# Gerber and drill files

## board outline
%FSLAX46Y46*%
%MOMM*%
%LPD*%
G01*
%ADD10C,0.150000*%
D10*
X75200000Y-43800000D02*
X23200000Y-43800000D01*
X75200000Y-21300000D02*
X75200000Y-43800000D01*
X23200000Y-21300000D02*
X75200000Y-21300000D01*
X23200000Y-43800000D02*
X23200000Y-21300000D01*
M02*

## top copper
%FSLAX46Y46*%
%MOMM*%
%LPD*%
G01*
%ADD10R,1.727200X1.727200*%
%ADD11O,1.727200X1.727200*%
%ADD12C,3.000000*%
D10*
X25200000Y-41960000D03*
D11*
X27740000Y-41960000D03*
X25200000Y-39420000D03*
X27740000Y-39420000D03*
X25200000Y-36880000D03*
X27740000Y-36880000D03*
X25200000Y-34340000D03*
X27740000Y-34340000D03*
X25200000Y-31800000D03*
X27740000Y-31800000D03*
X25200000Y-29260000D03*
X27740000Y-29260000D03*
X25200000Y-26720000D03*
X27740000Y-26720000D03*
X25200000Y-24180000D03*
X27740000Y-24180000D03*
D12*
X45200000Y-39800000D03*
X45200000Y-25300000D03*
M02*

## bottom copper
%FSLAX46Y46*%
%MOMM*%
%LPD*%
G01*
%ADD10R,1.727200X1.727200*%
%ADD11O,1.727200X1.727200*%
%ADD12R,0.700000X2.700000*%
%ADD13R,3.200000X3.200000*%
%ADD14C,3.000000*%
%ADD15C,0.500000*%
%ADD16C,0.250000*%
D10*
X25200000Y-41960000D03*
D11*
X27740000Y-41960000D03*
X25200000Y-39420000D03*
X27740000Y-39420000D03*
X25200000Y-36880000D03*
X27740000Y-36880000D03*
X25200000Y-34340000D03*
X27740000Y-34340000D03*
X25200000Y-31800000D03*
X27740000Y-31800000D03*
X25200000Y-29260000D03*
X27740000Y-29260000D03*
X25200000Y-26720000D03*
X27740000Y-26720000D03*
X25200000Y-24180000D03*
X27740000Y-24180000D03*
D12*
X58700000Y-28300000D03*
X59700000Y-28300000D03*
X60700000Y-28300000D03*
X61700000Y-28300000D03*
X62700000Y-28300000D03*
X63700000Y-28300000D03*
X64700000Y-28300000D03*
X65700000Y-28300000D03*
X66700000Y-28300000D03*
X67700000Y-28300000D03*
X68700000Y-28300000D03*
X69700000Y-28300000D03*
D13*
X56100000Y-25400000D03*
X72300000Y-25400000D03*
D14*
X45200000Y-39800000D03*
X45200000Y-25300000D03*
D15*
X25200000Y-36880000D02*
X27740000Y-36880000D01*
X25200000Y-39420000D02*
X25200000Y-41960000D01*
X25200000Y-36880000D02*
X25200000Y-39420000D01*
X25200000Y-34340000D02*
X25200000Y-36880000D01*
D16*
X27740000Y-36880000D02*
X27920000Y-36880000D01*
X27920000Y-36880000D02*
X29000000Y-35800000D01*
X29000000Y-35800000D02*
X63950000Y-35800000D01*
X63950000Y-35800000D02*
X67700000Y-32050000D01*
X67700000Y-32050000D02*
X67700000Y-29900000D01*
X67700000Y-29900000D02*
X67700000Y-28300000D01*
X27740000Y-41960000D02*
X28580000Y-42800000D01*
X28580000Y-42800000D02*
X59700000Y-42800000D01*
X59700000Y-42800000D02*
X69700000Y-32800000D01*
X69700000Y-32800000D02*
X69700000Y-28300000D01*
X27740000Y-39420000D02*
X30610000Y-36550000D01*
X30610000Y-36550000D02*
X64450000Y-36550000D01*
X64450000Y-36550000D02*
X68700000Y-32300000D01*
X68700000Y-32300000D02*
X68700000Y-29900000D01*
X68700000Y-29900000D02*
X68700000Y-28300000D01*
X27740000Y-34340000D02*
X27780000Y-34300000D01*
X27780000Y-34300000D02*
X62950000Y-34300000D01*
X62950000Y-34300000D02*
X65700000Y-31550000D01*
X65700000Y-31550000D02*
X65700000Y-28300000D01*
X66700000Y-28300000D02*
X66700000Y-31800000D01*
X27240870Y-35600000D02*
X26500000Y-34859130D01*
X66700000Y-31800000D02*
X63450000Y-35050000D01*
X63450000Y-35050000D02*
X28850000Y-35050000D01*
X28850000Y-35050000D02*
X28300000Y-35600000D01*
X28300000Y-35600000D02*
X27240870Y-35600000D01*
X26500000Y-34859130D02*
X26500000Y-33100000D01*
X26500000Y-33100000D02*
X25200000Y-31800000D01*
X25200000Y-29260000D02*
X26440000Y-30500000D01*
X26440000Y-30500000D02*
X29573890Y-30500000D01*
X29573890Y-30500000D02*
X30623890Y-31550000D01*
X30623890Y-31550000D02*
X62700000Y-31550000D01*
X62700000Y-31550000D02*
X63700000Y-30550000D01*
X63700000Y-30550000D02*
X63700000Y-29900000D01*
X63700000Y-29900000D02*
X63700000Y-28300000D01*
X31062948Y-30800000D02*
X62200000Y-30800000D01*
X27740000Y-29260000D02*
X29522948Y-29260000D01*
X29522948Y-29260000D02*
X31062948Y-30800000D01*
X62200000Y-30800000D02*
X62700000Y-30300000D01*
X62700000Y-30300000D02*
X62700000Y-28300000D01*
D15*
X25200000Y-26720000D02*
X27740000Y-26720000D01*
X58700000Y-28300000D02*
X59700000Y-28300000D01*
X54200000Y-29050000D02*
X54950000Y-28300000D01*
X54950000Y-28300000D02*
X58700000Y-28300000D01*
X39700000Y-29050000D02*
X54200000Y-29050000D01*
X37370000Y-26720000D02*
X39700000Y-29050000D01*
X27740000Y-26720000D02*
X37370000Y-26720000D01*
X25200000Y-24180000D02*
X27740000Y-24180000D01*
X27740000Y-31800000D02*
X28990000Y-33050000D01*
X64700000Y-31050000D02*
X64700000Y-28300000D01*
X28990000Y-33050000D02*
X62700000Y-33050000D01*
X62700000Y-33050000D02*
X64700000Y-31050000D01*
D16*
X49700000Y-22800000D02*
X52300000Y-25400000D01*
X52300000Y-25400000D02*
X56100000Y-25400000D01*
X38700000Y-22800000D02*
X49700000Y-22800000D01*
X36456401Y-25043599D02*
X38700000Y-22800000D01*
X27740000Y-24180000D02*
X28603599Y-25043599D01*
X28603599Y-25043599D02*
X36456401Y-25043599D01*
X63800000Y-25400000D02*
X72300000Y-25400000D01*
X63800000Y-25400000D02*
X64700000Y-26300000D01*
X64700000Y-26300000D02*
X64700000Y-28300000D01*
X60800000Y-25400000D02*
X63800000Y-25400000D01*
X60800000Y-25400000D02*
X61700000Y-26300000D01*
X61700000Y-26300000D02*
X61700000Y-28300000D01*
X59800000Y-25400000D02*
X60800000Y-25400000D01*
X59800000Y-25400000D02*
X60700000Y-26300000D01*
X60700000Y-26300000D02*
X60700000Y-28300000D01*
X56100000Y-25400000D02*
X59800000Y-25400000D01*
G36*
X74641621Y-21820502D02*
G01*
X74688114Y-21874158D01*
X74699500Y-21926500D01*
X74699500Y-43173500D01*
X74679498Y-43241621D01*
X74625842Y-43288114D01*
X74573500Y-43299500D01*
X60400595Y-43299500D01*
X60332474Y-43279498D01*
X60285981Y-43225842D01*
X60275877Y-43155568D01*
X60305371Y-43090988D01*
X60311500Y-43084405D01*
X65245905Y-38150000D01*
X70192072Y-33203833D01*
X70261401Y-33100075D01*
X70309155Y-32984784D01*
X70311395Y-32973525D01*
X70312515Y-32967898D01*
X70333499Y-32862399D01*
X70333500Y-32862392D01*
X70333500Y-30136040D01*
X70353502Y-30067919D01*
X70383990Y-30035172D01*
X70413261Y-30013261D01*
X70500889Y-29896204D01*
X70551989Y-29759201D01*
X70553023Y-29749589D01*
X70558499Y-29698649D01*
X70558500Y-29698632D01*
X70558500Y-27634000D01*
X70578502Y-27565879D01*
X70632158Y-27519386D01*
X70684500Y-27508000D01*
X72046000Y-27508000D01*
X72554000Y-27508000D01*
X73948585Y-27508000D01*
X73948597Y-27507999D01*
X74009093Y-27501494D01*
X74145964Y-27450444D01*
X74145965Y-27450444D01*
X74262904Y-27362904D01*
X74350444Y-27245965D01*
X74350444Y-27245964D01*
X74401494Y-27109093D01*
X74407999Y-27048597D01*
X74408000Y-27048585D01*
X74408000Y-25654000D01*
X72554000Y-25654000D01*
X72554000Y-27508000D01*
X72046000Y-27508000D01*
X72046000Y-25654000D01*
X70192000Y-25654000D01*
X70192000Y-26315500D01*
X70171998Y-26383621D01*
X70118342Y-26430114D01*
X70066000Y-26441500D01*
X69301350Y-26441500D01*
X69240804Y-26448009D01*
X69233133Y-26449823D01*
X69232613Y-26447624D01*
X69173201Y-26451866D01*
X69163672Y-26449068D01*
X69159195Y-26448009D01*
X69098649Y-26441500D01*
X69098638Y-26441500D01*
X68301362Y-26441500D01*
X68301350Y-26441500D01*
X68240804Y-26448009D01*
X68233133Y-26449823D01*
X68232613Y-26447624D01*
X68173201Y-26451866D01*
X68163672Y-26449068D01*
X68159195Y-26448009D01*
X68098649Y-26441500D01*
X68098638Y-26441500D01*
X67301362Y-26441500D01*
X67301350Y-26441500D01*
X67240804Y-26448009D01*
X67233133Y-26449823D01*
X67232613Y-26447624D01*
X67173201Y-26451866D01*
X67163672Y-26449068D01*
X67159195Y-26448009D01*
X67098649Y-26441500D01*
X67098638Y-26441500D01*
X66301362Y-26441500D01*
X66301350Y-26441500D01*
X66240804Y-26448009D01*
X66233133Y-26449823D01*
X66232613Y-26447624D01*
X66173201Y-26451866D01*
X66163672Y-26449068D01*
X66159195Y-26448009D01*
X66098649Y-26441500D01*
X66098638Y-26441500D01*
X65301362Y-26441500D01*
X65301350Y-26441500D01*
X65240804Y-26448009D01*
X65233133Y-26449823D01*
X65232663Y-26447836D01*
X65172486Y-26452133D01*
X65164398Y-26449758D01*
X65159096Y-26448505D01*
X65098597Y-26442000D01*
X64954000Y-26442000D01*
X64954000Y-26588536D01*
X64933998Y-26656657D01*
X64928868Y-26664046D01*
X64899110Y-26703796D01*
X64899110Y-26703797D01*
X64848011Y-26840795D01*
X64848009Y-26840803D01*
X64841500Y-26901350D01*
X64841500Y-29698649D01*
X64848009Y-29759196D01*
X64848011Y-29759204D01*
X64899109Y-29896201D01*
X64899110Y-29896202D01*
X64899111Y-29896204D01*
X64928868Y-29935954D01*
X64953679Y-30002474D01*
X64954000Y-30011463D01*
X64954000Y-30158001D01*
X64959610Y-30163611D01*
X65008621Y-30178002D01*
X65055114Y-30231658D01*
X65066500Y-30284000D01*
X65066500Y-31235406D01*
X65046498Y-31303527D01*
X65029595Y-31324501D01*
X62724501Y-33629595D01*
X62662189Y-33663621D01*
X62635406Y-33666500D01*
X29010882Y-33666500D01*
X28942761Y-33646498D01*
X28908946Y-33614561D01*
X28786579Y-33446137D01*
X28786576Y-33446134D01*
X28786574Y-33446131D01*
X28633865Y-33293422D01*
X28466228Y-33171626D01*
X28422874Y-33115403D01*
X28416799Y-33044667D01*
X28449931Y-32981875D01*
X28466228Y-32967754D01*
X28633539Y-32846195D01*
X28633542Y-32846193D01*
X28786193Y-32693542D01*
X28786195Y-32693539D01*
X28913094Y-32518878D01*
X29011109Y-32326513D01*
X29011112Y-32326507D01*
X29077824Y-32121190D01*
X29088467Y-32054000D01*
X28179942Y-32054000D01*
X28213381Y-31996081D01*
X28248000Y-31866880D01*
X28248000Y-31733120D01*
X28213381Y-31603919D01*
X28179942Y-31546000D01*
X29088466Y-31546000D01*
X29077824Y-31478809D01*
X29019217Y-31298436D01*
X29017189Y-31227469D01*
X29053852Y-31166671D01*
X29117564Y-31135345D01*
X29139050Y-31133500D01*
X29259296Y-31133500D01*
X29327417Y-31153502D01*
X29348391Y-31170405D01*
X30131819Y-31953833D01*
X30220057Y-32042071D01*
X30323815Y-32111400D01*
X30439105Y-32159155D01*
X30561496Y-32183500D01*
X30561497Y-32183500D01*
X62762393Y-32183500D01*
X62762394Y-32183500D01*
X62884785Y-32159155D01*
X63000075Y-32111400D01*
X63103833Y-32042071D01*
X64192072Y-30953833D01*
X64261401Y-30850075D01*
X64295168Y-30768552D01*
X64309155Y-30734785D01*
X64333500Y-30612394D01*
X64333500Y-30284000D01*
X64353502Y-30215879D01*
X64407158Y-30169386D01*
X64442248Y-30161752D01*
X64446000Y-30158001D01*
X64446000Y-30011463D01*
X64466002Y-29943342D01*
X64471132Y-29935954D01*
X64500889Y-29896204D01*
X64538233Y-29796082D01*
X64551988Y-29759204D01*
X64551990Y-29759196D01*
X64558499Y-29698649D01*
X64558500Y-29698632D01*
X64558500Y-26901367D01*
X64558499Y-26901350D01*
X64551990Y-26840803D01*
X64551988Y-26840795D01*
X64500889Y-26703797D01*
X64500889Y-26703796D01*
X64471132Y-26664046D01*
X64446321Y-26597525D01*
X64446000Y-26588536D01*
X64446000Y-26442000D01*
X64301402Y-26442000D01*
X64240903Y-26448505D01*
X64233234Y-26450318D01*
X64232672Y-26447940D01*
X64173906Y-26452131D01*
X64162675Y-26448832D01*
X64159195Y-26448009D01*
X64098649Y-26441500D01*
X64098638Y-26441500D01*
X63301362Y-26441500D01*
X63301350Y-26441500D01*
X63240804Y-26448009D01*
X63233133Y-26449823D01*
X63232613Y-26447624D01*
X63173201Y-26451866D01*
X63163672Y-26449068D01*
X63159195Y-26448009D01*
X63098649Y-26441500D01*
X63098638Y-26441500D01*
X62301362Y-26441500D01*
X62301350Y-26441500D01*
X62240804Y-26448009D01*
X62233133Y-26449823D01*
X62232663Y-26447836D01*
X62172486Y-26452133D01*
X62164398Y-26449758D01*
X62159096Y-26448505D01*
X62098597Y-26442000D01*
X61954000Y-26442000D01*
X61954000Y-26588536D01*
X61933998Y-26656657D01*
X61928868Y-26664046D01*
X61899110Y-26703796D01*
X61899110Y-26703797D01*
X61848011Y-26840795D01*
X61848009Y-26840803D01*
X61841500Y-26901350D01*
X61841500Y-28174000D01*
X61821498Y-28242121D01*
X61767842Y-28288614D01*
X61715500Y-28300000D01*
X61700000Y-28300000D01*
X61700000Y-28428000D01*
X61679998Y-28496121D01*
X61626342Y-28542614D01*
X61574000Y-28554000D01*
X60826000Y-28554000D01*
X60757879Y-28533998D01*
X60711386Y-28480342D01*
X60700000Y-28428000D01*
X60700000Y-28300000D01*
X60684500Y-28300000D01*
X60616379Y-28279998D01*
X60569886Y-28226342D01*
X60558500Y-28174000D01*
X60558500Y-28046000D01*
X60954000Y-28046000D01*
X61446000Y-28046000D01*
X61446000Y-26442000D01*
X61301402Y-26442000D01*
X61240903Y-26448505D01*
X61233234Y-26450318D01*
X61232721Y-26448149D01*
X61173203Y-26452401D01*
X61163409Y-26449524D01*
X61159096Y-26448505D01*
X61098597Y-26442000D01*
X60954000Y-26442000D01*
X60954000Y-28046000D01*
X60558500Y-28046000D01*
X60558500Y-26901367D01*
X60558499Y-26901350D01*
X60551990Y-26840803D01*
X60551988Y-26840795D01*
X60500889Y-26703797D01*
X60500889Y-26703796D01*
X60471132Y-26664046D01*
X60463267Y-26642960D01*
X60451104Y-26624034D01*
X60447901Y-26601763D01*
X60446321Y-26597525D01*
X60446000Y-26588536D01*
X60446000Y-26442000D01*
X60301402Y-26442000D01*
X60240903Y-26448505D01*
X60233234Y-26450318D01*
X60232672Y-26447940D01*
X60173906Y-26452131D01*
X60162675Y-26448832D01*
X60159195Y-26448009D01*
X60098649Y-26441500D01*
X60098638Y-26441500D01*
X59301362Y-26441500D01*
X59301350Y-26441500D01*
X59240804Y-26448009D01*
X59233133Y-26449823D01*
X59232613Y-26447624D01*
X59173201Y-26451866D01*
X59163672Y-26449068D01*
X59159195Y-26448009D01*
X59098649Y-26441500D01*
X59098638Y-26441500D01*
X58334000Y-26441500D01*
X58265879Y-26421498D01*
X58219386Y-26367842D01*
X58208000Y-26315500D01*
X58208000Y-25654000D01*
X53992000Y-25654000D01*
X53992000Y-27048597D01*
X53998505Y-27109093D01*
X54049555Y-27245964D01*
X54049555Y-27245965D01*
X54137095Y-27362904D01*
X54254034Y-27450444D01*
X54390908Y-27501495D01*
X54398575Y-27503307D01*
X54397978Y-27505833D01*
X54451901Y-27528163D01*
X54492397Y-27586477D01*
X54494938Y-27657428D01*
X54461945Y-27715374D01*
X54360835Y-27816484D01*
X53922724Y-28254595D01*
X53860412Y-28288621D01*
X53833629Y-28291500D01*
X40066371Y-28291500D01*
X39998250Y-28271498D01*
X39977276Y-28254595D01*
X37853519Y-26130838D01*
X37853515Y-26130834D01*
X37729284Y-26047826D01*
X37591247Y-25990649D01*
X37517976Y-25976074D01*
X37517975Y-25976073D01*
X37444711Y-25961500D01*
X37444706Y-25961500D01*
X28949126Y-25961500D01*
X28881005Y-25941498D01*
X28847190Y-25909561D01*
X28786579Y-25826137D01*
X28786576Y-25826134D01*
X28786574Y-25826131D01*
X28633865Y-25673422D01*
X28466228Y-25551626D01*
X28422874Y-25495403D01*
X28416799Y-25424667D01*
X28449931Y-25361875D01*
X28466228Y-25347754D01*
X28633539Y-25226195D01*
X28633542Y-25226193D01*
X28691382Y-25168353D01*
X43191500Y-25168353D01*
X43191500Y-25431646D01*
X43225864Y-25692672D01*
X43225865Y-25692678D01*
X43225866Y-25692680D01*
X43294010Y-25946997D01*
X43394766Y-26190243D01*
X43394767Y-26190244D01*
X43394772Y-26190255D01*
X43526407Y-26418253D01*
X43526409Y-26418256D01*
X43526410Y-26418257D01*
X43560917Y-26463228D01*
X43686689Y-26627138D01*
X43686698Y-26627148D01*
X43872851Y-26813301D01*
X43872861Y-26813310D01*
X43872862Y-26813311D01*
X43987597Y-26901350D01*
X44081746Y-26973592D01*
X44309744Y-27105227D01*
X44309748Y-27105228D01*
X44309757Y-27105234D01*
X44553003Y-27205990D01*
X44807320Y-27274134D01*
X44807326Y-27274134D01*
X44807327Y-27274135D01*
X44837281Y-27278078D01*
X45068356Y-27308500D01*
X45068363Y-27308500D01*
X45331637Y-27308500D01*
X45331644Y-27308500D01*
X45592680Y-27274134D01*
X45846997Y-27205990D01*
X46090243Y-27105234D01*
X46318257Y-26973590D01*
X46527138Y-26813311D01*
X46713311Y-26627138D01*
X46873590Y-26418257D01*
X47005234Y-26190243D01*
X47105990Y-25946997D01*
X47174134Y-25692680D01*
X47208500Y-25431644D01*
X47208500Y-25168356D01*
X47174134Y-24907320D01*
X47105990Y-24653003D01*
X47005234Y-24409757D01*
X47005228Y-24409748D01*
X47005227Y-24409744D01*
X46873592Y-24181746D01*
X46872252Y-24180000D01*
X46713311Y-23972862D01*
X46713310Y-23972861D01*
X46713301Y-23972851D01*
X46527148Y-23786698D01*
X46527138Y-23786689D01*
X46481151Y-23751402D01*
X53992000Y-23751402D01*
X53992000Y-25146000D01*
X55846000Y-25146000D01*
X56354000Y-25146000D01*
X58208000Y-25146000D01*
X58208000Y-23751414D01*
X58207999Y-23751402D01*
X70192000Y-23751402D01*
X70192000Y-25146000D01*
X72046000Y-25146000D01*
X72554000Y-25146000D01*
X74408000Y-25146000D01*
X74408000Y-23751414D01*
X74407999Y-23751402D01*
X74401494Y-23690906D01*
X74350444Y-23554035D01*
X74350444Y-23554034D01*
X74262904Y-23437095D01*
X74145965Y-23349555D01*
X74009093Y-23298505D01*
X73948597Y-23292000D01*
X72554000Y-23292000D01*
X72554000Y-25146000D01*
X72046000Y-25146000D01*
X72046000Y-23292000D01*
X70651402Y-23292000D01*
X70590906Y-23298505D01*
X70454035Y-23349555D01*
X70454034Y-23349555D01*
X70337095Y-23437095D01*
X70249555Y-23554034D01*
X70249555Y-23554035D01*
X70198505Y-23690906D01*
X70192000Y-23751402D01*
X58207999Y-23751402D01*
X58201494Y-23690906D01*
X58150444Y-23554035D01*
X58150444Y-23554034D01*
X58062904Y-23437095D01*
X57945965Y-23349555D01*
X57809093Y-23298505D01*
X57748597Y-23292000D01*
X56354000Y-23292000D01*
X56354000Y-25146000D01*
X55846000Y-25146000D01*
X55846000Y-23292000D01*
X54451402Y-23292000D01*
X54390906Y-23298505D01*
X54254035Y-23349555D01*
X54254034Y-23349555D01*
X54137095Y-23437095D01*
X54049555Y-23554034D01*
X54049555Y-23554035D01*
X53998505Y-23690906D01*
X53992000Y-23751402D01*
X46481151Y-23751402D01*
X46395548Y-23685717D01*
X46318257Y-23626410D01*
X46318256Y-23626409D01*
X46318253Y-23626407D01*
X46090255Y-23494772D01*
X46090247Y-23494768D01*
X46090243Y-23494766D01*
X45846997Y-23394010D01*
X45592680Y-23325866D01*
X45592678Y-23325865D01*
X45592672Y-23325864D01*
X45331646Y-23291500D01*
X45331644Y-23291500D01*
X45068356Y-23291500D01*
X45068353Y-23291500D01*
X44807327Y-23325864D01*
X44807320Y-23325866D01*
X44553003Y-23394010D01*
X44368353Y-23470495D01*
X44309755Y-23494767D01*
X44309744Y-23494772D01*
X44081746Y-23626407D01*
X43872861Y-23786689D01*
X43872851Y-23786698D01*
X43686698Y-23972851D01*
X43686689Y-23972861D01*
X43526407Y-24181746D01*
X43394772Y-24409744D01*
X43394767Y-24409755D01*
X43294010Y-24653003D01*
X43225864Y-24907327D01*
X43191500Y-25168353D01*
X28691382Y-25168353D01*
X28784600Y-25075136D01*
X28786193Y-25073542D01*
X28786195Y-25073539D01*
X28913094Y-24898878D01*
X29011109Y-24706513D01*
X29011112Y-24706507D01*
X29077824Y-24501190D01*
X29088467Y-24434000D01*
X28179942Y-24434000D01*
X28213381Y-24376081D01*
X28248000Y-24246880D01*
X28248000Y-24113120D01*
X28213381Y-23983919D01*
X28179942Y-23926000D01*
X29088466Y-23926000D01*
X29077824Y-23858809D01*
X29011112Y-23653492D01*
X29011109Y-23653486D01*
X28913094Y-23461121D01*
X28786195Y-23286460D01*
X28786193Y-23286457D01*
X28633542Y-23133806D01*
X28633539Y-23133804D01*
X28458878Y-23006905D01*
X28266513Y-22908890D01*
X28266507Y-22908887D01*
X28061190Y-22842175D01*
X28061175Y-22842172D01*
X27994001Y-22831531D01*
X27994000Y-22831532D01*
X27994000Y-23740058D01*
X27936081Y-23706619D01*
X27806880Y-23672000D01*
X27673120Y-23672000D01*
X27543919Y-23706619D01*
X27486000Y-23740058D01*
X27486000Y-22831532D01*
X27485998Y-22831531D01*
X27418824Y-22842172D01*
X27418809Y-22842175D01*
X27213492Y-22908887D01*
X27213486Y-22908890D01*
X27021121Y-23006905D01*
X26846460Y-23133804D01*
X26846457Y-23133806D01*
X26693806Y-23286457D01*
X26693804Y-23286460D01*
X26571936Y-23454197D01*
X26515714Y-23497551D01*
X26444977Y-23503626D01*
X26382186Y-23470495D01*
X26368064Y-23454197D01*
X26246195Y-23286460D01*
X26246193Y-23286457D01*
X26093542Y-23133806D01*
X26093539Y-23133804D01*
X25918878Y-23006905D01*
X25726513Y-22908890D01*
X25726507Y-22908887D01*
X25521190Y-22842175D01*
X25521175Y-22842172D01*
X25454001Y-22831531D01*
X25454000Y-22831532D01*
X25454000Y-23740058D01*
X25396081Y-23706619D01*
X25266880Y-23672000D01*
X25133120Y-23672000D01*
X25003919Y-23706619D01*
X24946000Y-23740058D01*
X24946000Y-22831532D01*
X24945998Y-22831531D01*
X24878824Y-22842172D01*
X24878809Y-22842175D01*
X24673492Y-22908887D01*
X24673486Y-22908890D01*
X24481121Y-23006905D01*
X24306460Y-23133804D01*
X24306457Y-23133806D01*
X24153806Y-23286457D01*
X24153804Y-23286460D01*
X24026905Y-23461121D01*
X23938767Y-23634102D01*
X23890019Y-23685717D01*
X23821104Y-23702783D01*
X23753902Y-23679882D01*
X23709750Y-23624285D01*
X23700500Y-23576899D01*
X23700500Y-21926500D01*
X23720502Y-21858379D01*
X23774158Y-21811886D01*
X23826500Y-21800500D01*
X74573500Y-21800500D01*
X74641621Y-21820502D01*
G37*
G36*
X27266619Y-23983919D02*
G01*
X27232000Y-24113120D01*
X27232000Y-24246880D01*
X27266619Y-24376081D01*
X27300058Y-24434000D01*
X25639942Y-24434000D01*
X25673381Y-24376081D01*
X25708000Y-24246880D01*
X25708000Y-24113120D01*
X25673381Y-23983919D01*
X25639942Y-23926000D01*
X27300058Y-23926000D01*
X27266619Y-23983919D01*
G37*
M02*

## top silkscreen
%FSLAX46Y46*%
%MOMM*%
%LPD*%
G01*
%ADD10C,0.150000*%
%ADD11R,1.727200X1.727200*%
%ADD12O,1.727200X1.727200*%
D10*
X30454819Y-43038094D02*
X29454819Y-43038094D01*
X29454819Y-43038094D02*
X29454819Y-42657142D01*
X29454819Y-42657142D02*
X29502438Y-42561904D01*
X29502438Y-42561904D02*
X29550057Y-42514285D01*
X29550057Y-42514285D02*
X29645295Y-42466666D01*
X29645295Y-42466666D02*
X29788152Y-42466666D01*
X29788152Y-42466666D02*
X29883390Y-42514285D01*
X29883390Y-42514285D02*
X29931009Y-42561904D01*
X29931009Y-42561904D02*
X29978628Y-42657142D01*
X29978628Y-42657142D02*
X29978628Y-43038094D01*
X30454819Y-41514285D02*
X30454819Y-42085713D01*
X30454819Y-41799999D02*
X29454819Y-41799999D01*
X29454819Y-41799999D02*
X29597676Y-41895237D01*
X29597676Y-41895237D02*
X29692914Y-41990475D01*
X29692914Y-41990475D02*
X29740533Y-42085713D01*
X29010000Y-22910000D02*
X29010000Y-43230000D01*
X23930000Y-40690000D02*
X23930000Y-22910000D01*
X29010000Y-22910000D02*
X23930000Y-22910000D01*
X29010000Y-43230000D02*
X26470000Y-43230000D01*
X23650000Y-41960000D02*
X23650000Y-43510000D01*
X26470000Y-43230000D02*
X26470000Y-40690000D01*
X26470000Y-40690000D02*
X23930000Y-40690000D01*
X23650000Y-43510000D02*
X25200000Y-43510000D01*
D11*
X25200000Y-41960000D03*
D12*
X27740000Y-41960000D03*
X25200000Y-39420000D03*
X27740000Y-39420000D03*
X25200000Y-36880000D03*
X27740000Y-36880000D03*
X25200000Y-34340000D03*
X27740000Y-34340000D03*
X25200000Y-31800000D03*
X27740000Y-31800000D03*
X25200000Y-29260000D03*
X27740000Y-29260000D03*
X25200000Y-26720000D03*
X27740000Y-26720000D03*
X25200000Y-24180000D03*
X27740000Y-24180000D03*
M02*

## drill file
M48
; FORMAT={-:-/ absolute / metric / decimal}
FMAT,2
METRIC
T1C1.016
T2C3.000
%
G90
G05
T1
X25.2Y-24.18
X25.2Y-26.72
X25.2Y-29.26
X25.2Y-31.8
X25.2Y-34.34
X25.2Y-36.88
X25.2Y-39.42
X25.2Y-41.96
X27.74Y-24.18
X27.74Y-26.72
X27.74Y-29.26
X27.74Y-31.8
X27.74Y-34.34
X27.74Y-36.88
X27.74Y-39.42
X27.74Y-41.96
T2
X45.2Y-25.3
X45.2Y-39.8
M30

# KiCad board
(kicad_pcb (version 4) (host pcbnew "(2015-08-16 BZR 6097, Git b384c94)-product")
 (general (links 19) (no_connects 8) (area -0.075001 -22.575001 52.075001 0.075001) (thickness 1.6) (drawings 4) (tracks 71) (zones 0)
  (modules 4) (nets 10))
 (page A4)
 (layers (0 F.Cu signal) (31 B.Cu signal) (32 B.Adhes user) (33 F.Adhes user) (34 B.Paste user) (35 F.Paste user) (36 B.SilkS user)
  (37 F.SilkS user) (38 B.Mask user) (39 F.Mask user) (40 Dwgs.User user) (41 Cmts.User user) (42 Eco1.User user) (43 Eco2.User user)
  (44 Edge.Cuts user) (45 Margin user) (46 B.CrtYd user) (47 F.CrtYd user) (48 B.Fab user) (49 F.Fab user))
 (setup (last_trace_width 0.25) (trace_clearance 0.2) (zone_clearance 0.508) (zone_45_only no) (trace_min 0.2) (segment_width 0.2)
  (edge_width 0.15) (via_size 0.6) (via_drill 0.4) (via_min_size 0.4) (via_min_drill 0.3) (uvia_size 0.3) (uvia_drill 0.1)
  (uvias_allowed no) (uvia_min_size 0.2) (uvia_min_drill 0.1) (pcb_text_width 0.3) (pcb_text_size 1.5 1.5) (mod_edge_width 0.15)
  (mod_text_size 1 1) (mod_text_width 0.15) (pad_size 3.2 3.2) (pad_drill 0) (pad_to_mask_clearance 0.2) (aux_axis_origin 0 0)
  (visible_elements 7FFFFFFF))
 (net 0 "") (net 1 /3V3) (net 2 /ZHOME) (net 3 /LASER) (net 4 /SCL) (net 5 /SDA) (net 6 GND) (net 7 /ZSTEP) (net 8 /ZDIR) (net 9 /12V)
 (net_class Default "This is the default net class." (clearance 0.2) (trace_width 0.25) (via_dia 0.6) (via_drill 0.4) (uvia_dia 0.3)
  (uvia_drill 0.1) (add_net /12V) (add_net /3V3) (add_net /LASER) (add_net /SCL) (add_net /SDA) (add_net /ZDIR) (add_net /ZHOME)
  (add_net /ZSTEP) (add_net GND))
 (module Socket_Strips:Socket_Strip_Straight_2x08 (layer F.Cu) (at 25.2 41.96 90)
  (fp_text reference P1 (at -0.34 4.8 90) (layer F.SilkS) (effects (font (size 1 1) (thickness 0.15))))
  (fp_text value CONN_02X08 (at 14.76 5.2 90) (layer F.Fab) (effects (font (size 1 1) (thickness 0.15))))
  (fp_line (start 19.05 3.81) (end -1.27 3.81) (layer F.SilkS) (width 0.15))
  (fp_line (start 1.27 -1.27) (end 19.05 -1.27) (layer F.SilkS) (width 0.15))
  (fp_line (start 19.05 3.81) (end 19.05 -1.27) (layer F.SilkS) (width 0.15))
  (fp_line (start -1.27 3.81) (end -1.27 1.27) (layer F.SilkS) (width 0.15))
  (fp_line (start 0 -1.55) (end -1.55 -1.55) (layer F.SilkS) (width 0.15))
  (fp_line (start -1.27 1.27) (end 1.27 1.27) (layer F.SilkS) (width 0.15))
  (fp_line (start 1.27 1.27) (end 1.27 -1.27) (layer F.SilkS) (width 0.15))
  (fp_line (start -1.55 -1.55) (end -1.55 0) (layer F.SilkS) (width 0.15))
  (pad 1 thru_hole rect (at 0 0 90) (size 1.7272 1.7272) (drill 1.016) (layers *.Cu *.Mask F.SilkS) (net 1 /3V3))
  (pad 2 thru_hole oval (at 0 2.54 90) (size 1.7272 1.7272) (drill 1.016) (layers *.Cu *.Mask F.SilkS) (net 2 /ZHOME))
  (pad 3 thru_hole oval (at 2.54 0 90) (size 1.7272 1.7272) (drill 1.016) (layers *.Cu *.Mask F.SilkS) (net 1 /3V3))
  (pad 4 thru_hole oval (at 2.54 2.54 90) (size 1.7272 1.7272) (drill 1.016) (layers *.Cu *.Mask F.SilkS) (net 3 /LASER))
  (pad 5 thru_hole oval (at 5.08 0 90) (size 1.7272 1.7272) (drill 1.016) (layers *.Cu *.Mask F.SilkS) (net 1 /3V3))
  (pad 6 thru_hole oval (at 5.08 2.54 90) (size 1.7272 1.7272) (drill 1.016) (layers *.Cu *.Mask F.SilkS) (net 1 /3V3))
  (pad 7 thru_hole oval (at 7.62 0 90) (size 1.7272 1.7272) (drill 1.016) (layers *.Cu *.Mask F.SilkS) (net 1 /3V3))
  (pad 8 thru_hole oval (at 7.62 2.54 90) (size 1.7272 1.7272) (drill 1.016) (layers *.Cu *.Mask F.SilkS) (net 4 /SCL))
  (pad 9 thru_hole oval (at 10.16 0 90) (size 1.7272 1.7272) (drill 1.016) (layers *.Cu *.Mask F.SilkS) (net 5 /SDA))
  (pad 10 thru_hole oval (at 10.16 2.54 90) (size 1.7272 1.7272) (drill 1.016) (layers *.Cu *.Mask F.SilkS) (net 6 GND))
  (pad 11 thru_hole oval (at 12.7 0 90) (size 1.7272 1.7272) (drill 1.016) (layers *.Cu *.Mask F.SilkS) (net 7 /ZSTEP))
  (pad 12 thru_hole oval (at 12.7 2.54 90) (size 1.7272 1.7272) (drill 1.016) (layers *.Cu *.Mask F.SilkS) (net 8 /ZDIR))
  (pad 13 thru_hole oval (at 15.24 0 90) (size 1.7272 1.7272) (drill 1.016) (layers *.Cu *.Mask F.SilkS) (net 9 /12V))
  (pad 14 thru_hole oval (at 15.24 2.54 90) (size 1.7272 1.7272) (drill 1.016) (layers *.Cu *.Mask F.SilkS) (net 9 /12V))
  (pad 15 thru_hole oval (at 17.78 0 90) (size 1.7272 1.7272) (drill 1.016) (layers *.Cu *.Mask F.SilkS) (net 6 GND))
  (pad 16 thru_hole oval (at 17.78 2.54 90) (size 1.7272 1.7272) (drill 1.016) (layers *.Cu *.Mask F.SilkS) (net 6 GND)))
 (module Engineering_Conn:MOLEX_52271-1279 (layer B.Cu) (at 64.2 28.3)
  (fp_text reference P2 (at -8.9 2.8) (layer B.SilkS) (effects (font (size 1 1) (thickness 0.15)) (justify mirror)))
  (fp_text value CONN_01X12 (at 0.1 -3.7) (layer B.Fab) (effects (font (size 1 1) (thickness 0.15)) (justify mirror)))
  (pad 1 smd rect (at -5.5 0) (size 0.7 2.7) (layers B.Cu B.Paste B.Mask) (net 9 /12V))
  (pad 2 smd rect (at -4.5 0) (size 0.7 2.7) (layers B.Cu B.Paste B.Mask) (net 9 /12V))
  (pad 3 smd rect (at -3.5 0) (size 0.7 2.7) (layers B.Cu B.Paste B.Mask) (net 6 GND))
  (pad 4 smd rect (at -2.5 0) (size 0.7 2.7) (layers B.Cu B.Paste B.Mask) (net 6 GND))
  (pad 5 smd rect (at -1.5 0) (size 0.7 2.7) (layers B.Cu B.Paste B.Mask) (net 8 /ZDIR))
  (pad 6 smd rect (at -0.5 0) (size 0.7 2.7) (layers B.Cu B.Paste B.Mask) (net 7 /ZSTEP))
  (pad 7 smd rect (at 0.5 0) (size 0.7 2.7) (layers B.Cu B.Paste B.Mask) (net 6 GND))
  (pad 8 smd rect (at 1.5 0) (size 0.7 2.7) (layers B.Cu B.Paste B.Mask) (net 4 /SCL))
  (pad 9 smd rect (at 2.5 0) (size 0.7 2.7) (layers B.Cu B.Paste B.Mask) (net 5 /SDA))
  (pad 10 smd rect (at 3.5 0) (size 0.7 2.7) (layers B.Cu B.Paste B.Mask) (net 1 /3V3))
  (pad 11 smd rect (at 4.5 0) (size 0.7 2.7) (layers B.Cu B.Paste B.Mask) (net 3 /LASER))
  (pad 12 smd rect (at 5.5 0) (size 0.7 2.7) (layers B.Cu B.Paste B.Mask) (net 2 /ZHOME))
  (pad 13 smd rect (at -8.1 -2.9) (size 3.2 3.2) (layers B.Cu B.Paste B.Mask) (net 6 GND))
  (pad 14 smd rect (at 8.1 -2.9) (size 3.2 3.2) (layers B.Cu B.Paste B.Mask) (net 6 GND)))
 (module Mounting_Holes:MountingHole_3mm (layer F.Cu) (at 45.2 39.8)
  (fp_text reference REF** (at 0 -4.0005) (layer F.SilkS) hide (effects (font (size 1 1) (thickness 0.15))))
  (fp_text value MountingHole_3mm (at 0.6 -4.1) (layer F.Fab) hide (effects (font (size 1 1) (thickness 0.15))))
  (pad 1 thru_hole circle (at 0 0) (size 3 3) (drill 3) (layers)))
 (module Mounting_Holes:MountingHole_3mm (layer F.Cu) (at 45.2 25.3)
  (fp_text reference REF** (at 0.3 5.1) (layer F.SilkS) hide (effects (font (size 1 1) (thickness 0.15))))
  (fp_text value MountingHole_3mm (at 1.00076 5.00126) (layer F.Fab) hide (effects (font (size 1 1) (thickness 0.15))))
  (pad 1 thru_hole circle (at 0 0) (size 3 3) (drill 3) (layers)))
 (gr_line (start 75.2 43.8) (end 23.2 43.8) (layer Edge.Cuts) (width 0.15))
 (gr_line (start 75.2 21.3) (end 75.2 43.8) (layer Edge.Cuts) (width 0.15))
 (gr_line (start 23.2 21.3) (end 75.2 21.3) (layer Edge.Cuts) (width 0.15))
 (gr_line (start 23.2 43.8) (end 23.2 21.3) (layer Edge.Cuts) (width 0.15))
 (segment (start 25.2 36.88) (end 27.74 36.88) (width 0.5) (layer B.Cu) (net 1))
 (segment (start 25.2 39.42) (end 25.2 41.96) (width 0.5) (layer B.Cu) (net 1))
 (segment (start 25.2 36.88) (end 25.2 39.42) (width 0.5) (layer B.Cu) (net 1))
 (segment (start 25.2 34.34) (end 25.2 36.88) (width 0.5) (layer B.Cu) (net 1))
 (segment (start 27.74 36.88) (end 27.92 36.88) (width 0.25) (layer B.Cu) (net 1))
 (segment (start 27.92 36.88) (end 29 35.8) (width 0.25) (layer B.Cu) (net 1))
 (segment (start 29 35.8) (end 63.95 35.8) (width 0.25) (layer B.Cu) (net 1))
 (segment (start 63.95 35.8) (end 67.7 32.05) (width 0.25) (layer B.Cu) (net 1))
 (segment (start 67.7 32.05) (end 67.7 29.9) (width 0.25) (layer B.Cu) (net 1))
 (segment (start 67.7 29.9) (end 67.7 28.3) (width 0.25) (layer B.Cu) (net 1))
 (segment (start 27.74 41.96) (end 28.58 42.8) (width 0.25) (layer B.Cu) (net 2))
 (segment (start 28.58 42.8) (end 59.7 42.8) (width 0.25) (layer B.Cu) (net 2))
 (segment (start 59.7 42.8) (end 69.7 32.8) (width 0.25) (layer B.Cu) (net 2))
 (segment (start 69.7 32.8) (end 69.7 28.3) (width 0.25) (layer B.Cu) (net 2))
 (segment (start 27.74 39.42) (end 30.61 36.55) (width 0.25) (layer B.Cu) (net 3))
 (segment (start 30.61 36.55) (end 64.45 36.55) (width 0.25) (layer B.Cu) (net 3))
 (segment (start 64.45 36.55) (end 68.7 32.3) (width 0.25) (layer B.Cu) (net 3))
 (segment (start 68.7 32.3) (end 68.7 29.9) (width 0.25) (layer B.Cu) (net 3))
 (segment (start 68.7 29.9) (end 68.7 28.3) (width 0.25) (layer B.Cu) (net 3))
 (segment (start 27.74 34.34) (end 27.78 34.3) (width 0.25) (layer B.Cu) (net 4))
 (segment (start 27.78 34.3) (end 62.95 34.3) (width 0.25) (layer B.Cu) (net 4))
 (segment (start 62.95 34.3) (end 65.7 31.55) (width 0.25) (layer B.Cu) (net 4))
 (segment (start 65.7 31.55) (end 65.7 28.3) (width 0.25) (layer B.Cu) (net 4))
 (segment (start 66.7 28.3) (end 66.7 31.8) (width 0.25) (layer B.Cu) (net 5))
 (segment (start 27.24087 35.6) (end 26.5 34.85913) (width 0.25) (layer B.Cu) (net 5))
 (segment (start 66.7 31.8) (end 63.45 35.05) (width 0.25) (layer B.Cu) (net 5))
 (segment (start 63.45 35.05) (end 28.85 35.05) (width 0.25) (layer B.Cu) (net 5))
 (segment (start 28.85 35.05) (end 28.3 35.6) (width 0.25) (layer B.Cu) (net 5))
 (segment (start 28.3 35.6) (end 27.24087 35.6) (width 0.25) (layer B.Cu) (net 5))
 (segment (start 26.5 34.85913) (end 26.5 33.1) (width 0.25) (layer B.Cu) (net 5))
 (segment (start 26.5 33.1) (end 25.2 31.8) (width 0.25) (layer B.Cu) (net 5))
 (segment (start 25.2 29.26) (end 26.44 30.5) (width 0.25) (layer B.Cu) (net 7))
 (segment (start 26.44 30.5) (end 29.57389 30.5) (width 0.25) (layer B.Cu) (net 7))
 (segment (start 29.57389 30.5) (end 30.62389 31.55) (width 0.25) (layer B.Cu) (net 7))
 (segment (start 30.62389 31.55) (end 62.7 31.55) (width 0.25) (layer B.Cu) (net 7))
 (segment (start 62.7 31.55) (end 63.7 30.55) (width 0.25) (layer B.Cu) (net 7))
 (segment (start 63.7 30.55) (end 63.7 29.9) (width 0.25) (layer B.Cu) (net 7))
 (segment (start 63.7 29.9) (end 63.7 28.3) (width 0.25) (layer B.Cu) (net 7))
 (segment (start 31.062948 30.8) (end 62.2 30.8) (width 0.25) (layer B.Cu) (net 8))
 (segment (start 27.74 29.26) (end 29.522948 29.26) (width 0.25) (layer B.Cu) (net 8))
 (segment (start 29.522948 29.26) (end 31.062948 30.8) (width 0.25) (layer B.Cu) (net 8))
 (segment (start 62.2 30.8) (end 62.7 30.3) (width 0.25) (layer B.Cu) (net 8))
 (segment (start 62.7 30.3) (end 62.7 28.3) (width 0.25) (layer B.Cu) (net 8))
 (segment (start 25.2 26.72) (end 27.74 26.72) (width 0.5) (layer B.Cu) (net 9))
 (segment (start 58.7 28.3) (end 59.7 28.3) (width 0.5) (layer B.Cu) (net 9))
 (segment (start 54.2 29.05) (end 54.95 28.3) (width 0.5) (layer B.Cu) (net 9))
 (segment (start 54.95 28.3) (end 58.7 28.3) (width 0.5) (layer B.Cu) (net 9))
 (segment (start 39.7 29.05) (end 54.2 29.05) (width 0.5) (layer B.Cu) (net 9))
 (segment (start 37.37 26.72) (end 39.7 29.05) (width 0.5) (layer B.Cu) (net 9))
 (segment (start 27.74 26.72) (end 37.37 26.72) (width 0.5) (layer B.Cu) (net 9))
 (segment (start 25.2 24.18) (end 27.74 24.18) (width 0.5) (layer B.Cu) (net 6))
 (segment (start 27.74 31.8) (end 28.99 33.05) (width 0.5) (layer B.Cu) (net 6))
 (segment (start 64.7 31.05) (end 64.7 28.3) (width 0.5) (layer B.Cu) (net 6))
 (segment (start 28.99 33.05) (end 62.7 33.05) (width 0.5) (layer B.Cu) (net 6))
 (segment (start 62.7 33.05) (end 64.7 31.05) (width 0.5) (layer B.Cu) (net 6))
 (segment (start 49.7 22.8) (end 52.3 25.4) (width 0.25) (layer B.Cu) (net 6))
 (segment (start 52.3 25.4) (end 56.1 25.4) (width 0.25) (layer B.Cu) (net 6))
 (segment (start 38.7 22.8) (end 49.7 22.8) (width 0.25) (layer B.Cu) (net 6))
 (segment (start 36.456401 25.043599) (end 38.7 22.8) (width 0.25) (layer B.Cu) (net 6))
 (segment (start 27.74 24.18) (end 28.603599 25.043599) (width 0.25) (layer B.Cu) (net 6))
 (segment (start 28.603599 25.043599) (end 36.456401 25.043599) (width 0.25) (layer B.Cu) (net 6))
 (segment (start 63.8 25.4) (end 72.3 25.4) (width 0.25) (layer B.Cu) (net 6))
 (segment (start 63.8 25.4) (end 64.7 26.3) (width 0.25) (layer B.Cu) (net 6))
 (segment (start 64.7 26.3) (end 64.7 28.3) (width 0.25) (layer B.Cu) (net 6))
 (segment (start 60.8 25.4) (end 63.8 25.4) (width 0.25) (layer B.Cu) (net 6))
 (segment (start 60.8 25.4) (end 61.7 26.3) (width 0.25) (layer B.Cu) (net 6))
 (segment (start 61.7 26.3) (end 61.7 28.3) (width 0.25) (layer B.Cu) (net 6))
 (segment (start 59.8 25.4) (end 60.8 25.4) (width 0.25) (layer B.Cu) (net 6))
 (segment (start 59.8 25.4) (end 60.7 26.3) (width 0.25) (layer B.Cu) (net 6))
 (segment (start 60.7 26.3) (end 60.7 28.3) (width 0.25) (layer B.Cu) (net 6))
 (segment (start 56.1 25.4) (end 59.8 25.4) (width 0.25) (layer B.Cu) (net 6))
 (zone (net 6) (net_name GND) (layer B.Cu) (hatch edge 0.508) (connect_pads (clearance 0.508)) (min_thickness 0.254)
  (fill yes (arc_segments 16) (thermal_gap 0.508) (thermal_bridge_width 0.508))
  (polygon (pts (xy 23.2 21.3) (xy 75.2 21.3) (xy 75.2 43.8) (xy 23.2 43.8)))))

